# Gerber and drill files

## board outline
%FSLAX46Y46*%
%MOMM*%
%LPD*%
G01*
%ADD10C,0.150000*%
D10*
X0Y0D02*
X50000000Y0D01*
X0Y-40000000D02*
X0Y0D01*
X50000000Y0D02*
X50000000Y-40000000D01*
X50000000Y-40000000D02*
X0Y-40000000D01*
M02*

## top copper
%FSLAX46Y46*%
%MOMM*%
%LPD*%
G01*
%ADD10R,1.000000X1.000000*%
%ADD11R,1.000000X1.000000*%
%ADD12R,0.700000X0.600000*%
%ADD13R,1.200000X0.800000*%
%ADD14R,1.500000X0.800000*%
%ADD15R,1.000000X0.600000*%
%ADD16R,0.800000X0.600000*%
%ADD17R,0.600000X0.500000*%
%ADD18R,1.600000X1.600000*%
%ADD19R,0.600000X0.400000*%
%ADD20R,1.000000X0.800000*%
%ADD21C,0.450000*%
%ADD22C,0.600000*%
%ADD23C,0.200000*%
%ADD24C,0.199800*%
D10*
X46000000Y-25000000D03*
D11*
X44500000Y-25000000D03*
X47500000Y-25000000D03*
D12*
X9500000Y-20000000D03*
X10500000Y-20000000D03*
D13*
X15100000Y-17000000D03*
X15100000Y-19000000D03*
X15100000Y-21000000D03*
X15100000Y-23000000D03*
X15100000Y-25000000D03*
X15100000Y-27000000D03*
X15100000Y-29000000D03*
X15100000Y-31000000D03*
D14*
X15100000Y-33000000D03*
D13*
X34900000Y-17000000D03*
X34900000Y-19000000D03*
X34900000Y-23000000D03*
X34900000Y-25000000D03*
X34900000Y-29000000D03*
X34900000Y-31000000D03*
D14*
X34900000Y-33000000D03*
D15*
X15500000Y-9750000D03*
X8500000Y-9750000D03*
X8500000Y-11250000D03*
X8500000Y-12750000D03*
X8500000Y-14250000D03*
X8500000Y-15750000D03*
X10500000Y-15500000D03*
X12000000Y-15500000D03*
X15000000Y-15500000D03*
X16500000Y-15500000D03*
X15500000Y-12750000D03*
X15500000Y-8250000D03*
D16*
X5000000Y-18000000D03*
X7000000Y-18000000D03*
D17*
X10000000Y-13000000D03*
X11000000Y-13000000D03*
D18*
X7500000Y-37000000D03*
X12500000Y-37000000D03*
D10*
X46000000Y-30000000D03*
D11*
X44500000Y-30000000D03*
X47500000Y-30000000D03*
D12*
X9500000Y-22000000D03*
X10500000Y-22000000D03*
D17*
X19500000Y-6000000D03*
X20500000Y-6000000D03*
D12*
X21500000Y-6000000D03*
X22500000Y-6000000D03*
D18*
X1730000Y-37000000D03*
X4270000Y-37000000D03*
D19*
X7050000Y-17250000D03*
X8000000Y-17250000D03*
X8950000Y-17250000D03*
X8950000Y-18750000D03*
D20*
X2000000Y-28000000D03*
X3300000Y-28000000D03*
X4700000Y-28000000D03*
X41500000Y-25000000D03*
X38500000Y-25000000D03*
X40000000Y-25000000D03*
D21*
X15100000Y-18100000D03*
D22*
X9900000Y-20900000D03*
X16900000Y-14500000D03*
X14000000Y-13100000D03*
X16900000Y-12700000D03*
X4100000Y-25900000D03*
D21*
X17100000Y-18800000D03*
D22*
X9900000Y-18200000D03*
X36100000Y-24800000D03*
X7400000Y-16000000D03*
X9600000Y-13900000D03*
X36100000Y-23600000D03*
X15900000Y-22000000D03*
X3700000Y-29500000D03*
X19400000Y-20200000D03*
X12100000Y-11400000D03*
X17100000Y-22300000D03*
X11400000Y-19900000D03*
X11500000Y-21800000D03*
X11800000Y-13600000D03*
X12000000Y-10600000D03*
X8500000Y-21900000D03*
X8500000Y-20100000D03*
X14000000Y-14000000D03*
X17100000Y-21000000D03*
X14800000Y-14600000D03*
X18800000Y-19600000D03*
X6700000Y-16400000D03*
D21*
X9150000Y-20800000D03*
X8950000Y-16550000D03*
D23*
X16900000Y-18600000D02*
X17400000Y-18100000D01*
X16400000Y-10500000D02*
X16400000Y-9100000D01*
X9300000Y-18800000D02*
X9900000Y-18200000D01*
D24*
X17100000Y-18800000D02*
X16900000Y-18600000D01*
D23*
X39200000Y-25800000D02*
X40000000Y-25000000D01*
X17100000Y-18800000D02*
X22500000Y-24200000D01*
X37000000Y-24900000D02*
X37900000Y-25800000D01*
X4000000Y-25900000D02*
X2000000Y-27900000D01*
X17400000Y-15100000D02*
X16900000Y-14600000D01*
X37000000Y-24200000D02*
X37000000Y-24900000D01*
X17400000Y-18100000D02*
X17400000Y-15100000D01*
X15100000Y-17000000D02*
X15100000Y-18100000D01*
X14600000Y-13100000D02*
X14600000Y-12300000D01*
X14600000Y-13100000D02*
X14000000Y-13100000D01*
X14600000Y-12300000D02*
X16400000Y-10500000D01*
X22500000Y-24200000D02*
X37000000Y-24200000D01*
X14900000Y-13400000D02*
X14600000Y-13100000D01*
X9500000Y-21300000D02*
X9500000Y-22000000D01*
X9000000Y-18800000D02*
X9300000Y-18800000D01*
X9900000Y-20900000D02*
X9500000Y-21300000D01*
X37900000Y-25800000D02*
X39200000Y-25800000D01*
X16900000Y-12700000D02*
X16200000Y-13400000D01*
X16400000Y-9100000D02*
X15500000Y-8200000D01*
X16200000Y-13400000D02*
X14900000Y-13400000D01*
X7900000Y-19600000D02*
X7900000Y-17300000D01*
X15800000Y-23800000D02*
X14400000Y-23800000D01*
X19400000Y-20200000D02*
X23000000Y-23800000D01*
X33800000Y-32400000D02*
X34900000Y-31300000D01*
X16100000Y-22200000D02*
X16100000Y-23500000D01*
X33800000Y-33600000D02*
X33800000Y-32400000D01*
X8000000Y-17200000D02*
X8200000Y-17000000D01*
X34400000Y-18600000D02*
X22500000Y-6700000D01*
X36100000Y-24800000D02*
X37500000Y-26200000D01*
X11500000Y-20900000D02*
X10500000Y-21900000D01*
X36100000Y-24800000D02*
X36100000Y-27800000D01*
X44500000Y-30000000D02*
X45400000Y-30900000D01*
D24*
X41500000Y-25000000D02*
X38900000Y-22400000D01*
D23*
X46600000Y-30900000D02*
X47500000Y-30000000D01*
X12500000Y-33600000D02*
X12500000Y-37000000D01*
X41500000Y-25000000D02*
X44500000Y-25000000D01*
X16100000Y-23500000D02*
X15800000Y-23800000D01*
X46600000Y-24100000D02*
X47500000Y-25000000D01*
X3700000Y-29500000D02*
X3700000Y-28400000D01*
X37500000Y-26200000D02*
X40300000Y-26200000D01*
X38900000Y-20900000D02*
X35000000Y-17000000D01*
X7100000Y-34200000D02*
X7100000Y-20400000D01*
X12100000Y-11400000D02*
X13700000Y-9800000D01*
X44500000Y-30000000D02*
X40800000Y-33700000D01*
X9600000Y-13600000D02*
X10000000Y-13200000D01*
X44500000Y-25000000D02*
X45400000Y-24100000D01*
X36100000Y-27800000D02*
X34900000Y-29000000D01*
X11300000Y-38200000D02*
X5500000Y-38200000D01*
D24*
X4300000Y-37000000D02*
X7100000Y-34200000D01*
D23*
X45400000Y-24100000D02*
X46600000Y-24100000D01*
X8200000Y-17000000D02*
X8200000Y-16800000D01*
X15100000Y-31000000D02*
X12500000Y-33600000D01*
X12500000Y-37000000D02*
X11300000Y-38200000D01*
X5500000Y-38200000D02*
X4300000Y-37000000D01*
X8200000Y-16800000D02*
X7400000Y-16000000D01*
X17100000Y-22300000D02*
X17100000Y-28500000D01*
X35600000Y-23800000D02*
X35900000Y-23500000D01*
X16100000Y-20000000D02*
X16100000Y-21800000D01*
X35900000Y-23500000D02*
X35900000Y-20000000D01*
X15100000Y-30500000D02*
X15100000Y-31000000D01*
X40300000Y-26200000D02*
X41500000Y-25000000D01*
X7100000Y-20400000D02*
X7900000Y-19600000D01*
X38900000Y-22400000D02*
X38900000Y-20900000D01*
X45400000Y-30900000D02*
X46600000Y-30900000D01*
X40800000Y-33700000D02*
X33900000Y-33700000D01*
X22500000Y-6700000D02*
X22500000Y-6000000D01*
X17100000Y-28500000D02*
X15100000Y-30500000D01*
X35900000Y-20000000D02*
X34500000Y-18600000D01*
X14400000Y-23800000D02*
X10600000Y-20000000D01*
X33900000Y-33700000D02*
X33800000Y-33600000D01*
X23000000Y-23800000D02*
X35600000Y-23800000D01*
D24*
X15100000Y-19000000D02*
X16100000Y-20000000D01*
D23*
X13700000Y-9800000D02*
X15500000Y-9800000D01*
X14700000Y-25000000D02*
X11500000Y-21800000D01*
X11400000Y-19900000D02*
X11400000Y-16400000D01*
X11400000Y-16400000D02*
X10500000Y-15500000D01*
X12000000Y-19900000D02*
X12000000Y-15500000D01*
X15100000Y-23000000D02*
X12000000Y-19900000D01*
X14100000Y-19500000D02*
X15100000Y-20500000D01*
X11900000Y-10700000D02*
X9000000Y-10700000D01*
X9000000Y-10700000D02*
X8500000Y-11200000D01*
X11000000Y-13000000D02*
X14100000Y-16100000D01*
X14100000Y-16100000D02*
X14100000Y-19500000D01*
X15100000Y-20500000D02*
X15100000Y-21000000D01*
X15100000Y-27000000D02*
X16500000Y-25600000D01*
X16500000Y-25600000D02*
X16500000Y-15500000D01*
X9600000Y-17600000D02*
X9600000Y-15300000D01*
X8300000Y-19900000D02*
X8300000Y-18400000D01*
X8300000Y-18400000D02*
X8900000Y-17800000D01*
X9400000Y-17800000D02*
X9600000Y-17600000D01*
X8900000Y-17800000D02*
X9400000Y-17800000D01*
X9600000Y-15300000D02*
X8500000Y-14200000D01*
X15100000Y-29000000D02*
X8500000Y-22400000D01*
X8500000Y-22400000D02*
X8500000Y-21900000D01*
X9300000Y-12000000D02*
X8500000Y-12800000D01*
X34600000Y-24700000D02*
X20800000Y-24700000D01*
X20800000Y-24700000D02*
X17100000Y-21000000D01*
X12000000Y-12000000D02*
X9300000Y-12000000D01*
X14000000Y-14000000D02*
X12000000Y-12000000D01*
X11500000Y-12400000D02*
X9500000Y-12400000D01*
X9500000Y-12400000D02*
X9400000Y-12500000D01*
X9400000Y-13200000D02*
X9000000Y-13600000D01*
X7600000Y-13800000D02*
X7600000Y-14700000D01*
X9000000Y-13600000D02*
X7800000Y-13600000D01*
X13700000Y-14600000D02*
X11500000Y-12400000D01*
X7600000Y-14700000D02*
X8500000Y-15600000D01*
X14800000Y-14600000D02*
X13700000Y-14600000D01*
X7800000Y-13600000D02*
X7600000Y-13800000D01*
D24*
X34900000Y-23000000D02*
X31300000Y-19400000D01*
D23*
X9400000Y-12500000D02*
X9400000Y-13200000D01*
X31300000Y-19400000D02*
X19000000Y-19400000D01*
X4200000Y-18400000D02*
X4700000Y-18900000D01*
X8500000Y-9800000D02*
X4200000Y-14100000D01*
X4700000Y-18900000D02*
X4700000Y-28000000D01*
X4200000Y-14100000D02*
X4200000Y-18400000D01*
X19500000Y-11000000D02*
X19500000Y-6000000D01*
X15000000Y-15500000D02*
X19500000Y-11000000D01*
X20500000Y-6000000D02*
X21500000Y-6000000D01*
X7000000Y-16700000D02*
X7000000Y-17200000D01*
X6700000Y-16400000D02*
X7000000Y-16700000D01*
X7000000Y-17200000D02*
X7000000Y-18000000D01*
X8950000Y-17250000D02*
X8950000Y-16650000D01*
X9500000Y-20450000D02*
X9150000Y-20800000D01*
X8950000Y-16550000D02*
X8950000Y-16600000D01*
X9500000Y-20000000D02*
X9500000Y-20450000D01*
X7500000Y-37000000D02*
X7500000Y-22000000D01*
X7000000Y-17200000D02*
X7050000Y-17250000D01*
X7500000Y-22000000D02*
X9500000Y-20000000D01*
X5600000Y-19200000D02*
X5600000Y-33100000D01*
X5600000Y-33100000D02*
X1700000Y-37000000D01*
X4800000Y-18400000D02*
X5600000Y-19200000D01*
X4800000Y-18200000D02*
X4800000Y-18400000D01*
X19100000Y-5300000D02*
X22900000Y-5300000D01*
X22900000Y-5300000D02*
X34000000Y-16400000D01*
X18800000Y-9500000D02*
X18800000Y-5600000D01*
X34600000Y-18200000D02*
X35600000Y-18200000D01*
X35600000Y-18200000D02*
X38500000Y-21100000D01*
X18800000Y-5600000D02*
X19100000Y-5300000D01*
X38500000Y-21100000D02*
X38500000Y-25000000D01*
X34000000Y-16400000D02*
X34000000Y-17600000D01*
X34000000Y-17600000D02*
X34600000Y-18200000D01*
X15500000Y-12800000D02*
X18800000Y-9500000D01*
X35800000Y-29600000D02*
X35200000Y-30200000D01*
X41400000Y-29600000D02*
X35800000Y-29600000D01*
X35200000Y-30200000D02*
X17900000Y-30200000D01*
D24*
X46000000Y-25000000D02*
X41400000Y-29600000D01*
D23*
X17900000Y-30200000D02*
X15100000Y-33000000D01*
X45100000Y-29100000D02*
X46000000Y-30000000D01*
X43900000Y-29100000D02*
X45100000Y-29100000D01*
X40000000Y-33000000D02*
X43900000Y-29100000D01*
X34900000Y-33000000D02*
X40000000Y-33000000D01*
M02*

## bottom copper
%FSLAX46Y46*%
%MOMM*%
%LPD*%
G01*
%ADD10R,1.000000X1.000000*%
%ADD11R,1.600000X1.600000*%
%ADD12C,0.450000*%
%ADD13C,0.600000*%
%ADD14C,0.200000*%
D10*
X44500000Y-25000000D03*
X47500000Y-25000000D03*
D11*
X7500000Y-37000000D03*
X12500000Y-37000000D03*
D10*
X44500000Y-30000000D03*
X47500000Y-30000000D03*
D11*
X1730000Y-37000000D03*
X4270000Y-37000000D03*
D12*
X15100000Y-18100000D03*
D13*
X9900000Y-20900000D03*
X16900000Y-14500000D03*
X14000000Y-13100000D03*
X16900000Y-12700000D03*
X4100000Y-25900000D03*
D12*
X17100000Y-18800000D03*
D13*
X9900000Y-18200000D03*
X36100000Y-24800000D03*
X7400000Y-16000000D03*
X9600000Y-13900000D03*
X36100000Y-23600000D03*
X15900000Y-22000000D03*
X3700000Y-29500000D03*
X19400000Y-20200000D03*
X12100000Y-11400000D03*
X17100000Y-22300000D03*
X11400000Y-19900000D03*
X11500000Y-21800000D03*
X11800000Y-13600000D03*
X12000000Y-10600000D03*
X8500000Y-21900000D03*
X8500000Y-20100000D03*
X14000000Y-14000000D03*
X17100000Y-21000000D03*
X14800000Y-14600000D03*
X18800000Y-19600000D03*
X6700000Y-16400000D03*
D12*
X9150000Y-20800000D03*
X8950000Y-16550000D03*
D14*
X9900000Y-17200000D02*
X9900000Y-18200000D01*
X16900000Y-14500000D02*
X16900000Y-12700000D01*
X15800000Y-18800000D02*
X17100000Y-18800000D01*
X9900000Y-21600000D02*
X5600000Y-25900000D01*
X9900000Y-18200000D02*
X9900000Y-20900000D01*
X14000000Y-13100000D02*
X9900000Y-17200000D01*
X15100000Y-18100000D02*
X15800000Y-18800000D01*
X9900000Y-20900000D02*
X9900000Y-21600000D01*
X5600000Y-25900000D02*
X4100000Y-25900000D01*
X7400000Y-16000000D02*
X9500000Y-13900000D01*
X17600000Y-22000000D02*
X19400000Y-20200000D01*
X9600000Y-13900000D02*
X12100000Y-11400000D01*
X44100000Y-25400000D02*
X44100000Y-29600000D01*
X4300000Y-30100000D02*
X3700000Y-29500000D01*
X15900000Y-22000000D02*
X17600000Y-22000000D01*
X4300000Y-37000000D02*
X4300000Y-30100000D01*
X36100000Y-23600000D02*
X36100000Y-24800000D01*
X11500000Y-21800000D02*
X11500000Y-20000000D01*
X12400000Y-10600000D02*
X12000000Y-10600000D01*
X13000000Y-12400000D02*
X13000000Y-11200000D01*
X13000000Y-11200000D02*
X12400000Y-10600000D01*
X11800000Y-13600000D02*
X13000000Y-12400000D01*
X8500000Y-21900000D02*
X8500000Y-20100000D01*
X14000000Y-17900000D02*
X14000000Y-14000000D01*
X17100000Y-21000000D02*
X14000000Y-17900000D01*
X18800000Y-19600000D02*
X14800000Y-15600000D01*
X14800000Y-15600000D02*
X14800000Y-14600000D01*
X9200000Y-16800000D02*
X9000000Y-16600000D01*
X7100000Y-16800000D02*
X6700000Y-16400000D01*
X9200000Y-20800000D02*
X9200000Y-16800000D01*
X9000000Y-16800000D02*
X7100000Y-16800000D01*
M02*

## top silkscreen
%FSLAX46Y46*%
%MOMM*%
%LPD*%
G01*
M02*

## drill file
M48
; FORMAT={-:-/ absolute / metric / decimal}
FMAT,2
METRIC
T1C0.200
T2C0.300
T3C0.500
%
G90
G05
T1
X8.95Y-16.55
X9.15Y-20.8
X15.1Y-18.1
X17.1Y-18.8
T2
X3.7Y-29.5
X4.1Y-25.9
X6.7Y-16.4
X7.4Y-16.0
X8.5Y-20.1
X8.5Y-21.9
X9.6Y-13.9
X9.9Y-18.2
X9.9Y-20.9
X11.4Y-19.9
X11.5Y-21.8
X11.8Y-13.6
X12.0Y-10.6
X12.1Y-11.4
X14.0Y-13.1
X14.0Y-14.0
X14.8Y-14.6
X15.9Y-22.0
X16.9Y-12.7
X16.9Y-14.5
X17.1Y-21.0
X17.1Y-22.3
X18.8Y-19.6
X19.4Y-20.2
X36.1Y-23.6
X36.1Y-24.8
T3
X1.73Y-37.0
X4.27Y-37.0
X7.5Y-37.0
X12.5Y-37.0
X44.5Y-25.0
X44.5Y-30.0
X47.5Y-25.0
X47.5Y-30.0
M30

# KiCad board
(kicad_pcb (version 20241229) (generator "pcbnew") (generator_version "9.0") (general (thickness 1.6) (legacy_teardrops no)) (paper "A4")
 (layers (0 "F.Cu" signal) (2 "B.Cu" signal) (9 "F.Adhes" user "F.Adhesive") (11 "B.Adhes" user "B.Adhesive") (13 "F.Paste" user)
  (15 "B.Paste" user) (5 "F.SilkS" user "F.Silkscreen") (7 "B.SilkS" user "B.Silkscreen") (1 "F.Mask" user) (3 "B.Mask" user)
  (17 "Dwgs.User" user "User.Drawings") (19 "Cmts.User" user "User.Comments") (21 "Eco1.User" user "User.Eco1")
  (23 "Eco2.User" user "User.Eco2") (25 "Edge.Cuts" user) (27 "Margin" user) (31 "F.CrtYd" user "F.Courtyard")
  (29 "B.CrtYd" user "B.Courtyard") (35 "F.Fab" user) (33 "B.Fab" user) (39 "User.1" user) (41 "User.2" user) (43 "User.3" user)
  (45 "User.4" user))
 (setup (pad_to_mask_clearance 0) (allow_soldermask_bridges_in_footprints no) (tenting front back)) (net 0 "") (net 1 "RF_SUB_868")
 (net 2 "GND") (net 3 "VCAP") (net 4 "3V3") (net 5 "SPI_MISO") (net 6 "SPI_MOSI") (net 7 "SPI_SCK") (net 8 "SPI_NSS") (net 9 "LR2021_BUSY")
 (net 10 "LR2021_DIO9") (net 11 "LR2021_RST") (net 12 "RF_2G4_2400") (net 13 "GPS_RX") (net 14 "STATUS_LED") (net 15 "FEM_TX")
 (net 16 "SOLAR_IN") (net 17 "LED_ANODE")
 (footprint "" (layer "F.Cu") (at 46 25)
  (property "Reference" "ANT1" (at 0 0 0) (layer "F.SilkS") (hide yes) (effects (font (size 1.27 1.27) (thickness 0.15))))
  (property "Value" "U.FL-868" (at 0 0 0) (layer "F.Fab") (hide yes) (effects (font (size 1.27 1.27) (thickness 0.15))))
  (pad "1" smd rect (at 0 0) (size 1 1) (layers "F.Cu" "F.Mask") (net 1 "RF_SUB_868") (thermal_bridge_angle 45))
  (pad "2" thru_hole rect (at -1.5 0) (size 1 1) (drill 0.5) (layers "*.Cu" "*.Mask") (remove_unused_layers no) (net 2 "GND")
   (thermal_bridge_angle 45))
  (pad "3" thru_hole rect (at 1.5 0) (size 1 1) (drill 0.5) (layers "*.Cu" "*.Mask") (remove_unused_layers no) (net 2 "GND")
   (thermal_bridge_angle 45)))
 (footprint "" (layer "F.Cu") (at 10 20)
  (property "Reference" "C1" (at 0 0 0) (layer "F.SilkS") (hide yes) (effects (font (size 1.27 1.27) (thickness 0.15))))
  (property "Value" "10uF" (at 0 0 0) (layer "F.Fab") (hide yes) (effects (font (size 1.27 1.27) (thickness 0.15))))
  (pad "1" smd rect (at -0.5 0) (size 0.7 0.6) (layers "F.Cu" "F.Mask") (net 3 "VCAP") (thermal_bridge_angle 45))
  (pad "2" smd rect (at 0.5 0) (size 0.7 0.6) (layers "F.Cu" "F.Mask") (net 2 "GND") (thermal_bridge_angle 45)))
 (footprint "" (layer "F.Cu") (at 25 25)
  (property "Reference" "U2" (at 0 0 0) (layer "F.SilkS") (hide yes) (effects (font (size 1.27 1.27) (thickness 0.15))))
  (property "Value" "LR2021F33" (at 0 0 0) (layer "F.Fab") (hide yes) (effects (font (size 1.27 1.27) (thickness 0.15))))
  (pad "1" smd rect (at -9.9 -8) (size 1.2 0.8) (layers "F.Cu" "F.Mask") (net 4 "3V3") (thermal_bridge_angle 45))
  (pad "2" smd rect (at -9.9 -6) (size 1.2 0.8) (layers "F.Cu" "F.Mask") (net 2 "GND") (thermal_bridge_angle 45))
  (pad "3" smd rect (at -9.9 -4) (size 1.2 0.8) (layers "F.Cu" "F.Mask") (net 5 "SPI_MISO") (thermal_bridge_angle 45))
  (pad "4" smd rect (at -9.9 -2) (size 1.2 0.8) (layers "F.Cu" "F.Mask") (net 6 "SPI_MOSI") (thermal_bridge_angle 45))
  (pad "5" smd rect (at -9.9 0) (size 1.2 0.8) (layers "F.Cu" "F.Mask") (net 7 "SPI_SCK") (thermal_bridge_angle 45))
  (pad "6" smd rect (at -9.9 2) (size 1.2 0.8) (layers "F.Cu" "F.Mask") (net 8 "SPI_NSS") (thermal_bridge_angle 45))
  (pad "7" smd rect (at -9.9 4) (size 1.2 0.8) (layers "F.Cu" "F.Mask") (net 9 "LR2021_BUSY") (thermal_bridge_angle 45))
  (pad "8" smd rect (at -9.9 6) (size 1.2 0.8) (layers "F.Cu" "F.Mask") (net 2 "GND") (thermal_bridge_angle 45))
  (pad "9" smd rect (at -9.9 8) (size 1.5 0.8) (layers "F.Cu" "F.Mask") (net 1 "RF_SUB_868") (thermal_bridge_angle 45))
  (pad "10" smd rect (at 9.9 -8) (size 1.2 0.8) (layers "F.Cu" "F.Mask") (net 2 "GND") (thermal_bridge_angle 45))
  (pad "11" smd rect (at 9.9 -6) (size 1.2 0.8) (layers "F.Cu" "F.Mask") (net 2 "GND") (thermal_bridge_angle 45))
  (pad "13" smd rect (at 9.9 -2) (size 1.2 0.8) (layers "F.Cu" "F.Mask") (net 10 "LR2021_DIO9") (thermal_bridge_angle 45))
  (pad "14" smd rect (at 9.9 0) (size 1.2 0.8) (layers "F.Cu" "F.Mask") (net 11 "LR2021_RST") (thermal_bridge_angle 45))
  (pad "16" smd rect (at 9.9 4) (size 1.2 0.8) (layers "F.Cu" "F.Mask") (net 2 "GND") (thermal_bridge_angle 45))
  (pad "17" smd rect (at 9.9 6) (size 1.2 0.8) (layers "F.Cu" "F.Mask") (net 2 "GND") (thermal_bridge_angle 45))
  (pad "18" smd rect (at 9.9 8) (size 1.5 0.8) (layers "F.Cu" "F.Mask") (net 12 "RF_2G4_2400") (thermal_bridge_angle 45)))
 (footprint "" (layer "F.Cu") (at 12 12)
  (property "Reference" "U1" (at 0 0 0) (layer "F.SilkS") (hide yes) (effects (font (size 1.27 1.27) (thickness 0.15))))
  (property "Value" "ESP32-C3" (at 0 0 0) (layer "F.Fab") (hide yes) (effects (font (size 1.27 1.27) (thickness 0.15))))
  (pad "GND" smd rect (at 3.5 -2.25) (size 1 0.6) (layers "F.Cu" "F.Mask") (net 2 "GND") (thermal_bridge_angle 45))
  (pad "GPIO1" smd rect (at -3.5 -2.25) (size 1 0.6) (layers "F.Cu" "F.Mask") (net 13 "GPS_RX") (thermal_bridge_angle 45))
  (pad "GPIO2" smd rect (at -3.5 -0.75) (size 1 0.6) (layers "F.Cu" "F.Mask") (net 5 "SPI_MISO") (thermal_bridge_angle 45))
  (pad "GPIO3" smd rect (at -3.5 0.75) (size 1 0.6) (layers "F.Cu" "F.Mask") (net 11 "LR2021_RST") (thermal_bridge_angle 45))
  (pad "GPIO4" smd rect (at -3.5 2.25) (size 1 0.6) (layers "F.Cu" "F.Mask") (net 9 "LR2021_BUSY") (thermal_bridge_angle 45))
  (pad "GPIO5" smd rect (at -3.5 3.75) (size 1 0.6) (layers "F.Cu" "F.Mask") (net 10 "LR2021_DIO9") (thermal_bridge_angle 45))
  (pad "GPIO6" smd rect (at -1.5 3.5) (size 1 0.6) (layers "F.Cu" "F.Mask") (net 7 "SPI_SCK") (thermal_bridge_angle 45))
  (pad "GPIO7" smd rect (at 0 3.5) (size 1 0.6) (layers "F.Cu" "F.Mask") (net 6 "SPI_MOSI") (thermal_bridge_angle 45))
  (pad "GPIO9" smd rect (at 3 3.5) (size 1 0.6) (layers "F.Cu" "F.Mask") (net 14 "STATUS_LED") (thermal_bridge_angle 45))
  (pad "GPIO10" smd rect (at 4.5 3.5) (size 1 0.6) (layers "F.Cu" "F.Mask") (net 8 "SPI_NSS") (thermal_bridge_angle 45))
  (pad "GPIO19" smd rect (at 3.5 0.75) (size 1 0.6) (layers "F.Cu" "F.Mask") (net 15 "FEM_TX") (thermal_bridge_angle 45))
  (pad "VCC" smd rect (at 3.5 -3.75) (size 1 0.6) (layers "F.Cu" "F.Mask") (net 4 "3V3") (thermal_bridge_angle 45)))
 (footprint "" (layer "F.Cu") (at 6 18)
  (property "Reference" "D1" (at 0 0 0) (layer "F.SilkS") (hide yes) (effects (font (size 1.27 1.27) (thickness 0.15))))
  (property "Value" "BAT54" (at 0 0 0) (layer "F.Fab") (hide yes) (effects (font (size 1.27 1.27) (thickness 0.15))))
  (pad "A" smd rect (at -1 0) (size 0.8 0.6) (layers "F.Cu" "F.Mask") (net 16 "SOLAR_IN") (thermal_bridge_angle 45))
  (pad "K" smd rect (at 1 0) (size 0.8 0.6) (layers "F.Cu" "F.Mask") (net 3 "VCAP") (thermal_bridge_angle 45)))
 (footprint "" (layer "F.Cu") (at 10.5 13)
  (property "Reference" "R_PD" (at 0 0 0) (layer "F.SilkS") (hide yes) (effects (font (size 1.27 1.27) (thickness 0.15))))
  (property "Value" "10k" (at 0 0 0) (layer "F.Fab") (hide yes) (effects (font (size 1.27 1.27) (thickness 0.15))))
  (pad "1" smd rect (at -0.5 0) (size 0.6 0.5) (layers "F.Cu" "F.Mask") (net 2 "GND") (thermal_bridge_angle 45))
  (pad "2" smd rect (at 0.5 0) (size 0.6 0.5) (layers "F.Cu" "F.Mask") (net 5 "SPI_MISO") (thermal_bridge_angle 45)))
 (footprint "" (layer "F.Cu") (at 10 37)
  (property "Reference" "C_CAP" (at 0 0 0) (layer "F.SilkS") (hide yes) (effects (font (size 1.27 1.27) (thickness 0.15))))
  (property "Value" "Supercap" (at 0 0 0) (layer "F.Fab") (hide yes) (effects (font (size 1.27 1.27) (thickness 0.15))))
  (pad "1" thru_hole rect (at -2.5 0) (size 1.6 1.6) (drill 0.5) (layers "*.Cu" "*.Mask") (remove_unused_layers no) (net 3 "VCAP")
   (thermal_bridge_angle 45))
  (pad "2" thru_hole rect (at 2.5 0) (size 1.6 1.6) (drill 0.5) (layers "*.Cu" "*.Mask") (remove_unused_layers no) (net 2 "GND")
   (thermal_bridge_angle 45)))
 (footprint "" (layer "F.Cu") (at 46 30)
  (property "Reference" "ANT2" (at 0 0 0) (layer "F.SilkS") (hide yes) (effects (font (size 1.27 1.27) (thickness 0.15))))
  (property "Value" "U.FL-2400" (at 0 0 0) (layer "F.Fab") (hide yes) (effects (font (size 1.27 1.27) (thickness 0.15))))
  (pad "1" smd rect (at 0 0) (size 1 1) (layers "F.Cu" "F.Mask") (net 12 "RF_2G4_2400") (thermal_bridge_angle 45))
  (pad "2" thru_hole rect (at -1.5 0) (size 1 1) (drill 0.5) (layers "*.Cu" "*.Mask") (remove_unused_layers no) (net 2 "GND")
   (thermal_bridge_angle 45))
  (pad "3" thru_hole rect (at 1.5 0) (size 1 1) (drill 0.5) (layers "*.Cu" "*.Mask") (remove_unused_layers no) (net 2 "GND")
   (thermal_bridge_angle 45)))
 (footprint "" (layer "F.Cu") (at 10 22)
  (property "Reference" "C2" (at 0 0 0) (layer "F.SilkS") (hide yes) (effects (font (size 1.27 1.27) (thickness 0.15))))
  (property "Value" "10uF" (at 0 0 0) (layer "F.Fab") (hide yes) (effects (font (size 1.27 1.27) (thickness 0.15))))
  (pad "1" smd rect (at -0.5 0) (size 0.7 0.6) (layers "F.Cu" "F.Mask") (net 4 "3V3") (thermal_bridge_angle 45))
  (pad "2" smd rect (at 0.5 0) (size 0.7 0.6) (layers "F.Cu" "F.Mask") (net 2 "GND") (thermal_bridge_angle 45)))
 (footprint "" (layer "F.Cu") (at 20 6)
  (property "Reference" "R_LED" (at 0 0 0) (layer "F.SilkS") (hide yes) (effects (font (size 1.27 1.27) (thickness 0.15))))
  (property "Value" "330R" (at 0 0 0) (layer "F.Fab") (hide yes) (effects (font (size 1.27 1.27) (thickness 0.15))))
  (pad "1" smd rect (at -0.5 0) (size 0.6 0.5) (layers "F.Cu" "F.Mask") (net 14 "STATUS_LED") (thermal_bridge_angle 45))
  (pad "2" smd rect (at 0.5 0) (size 0.6 0.5) (layers "F.Cu" "F.Mask") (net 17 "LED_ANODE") (thermal_bridge_angle 45)))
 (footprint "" (layer "F.Cu") (at 22 6)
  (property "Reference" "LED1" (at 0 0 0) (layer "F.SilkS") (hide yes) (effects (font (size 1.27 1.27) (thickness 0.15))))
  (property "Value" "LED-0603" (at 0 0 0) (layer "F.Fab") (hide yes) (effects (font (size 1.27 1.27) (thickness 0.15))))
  (pad "A" smd rect (at -0.5 0) (size 0.7 0.6) (layers "F.Cu" "F.Mask") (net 17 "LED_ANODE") (thermal_bridge_angle 45))
  (pad "K" smd rect (at 0.5 0) (size 0.7 0.6) (layers "F.Cu" "F.Mask") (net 2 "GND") (thermal_bridge_angle 45)))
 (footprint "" (layer "F.Cu") (at 3 37)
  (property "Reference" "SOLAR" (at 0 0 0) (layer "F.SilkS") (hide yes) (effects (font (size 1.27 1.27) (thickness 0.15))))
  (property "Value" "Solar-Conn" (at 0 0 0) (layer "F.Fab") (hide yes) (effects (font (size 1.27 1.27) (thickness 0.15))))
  (pad "1" thru_hole rect (at -1.27 0) (size 1.6 1.6) (drill 0.5) (layers "*.Cu" "*.Mask") (remove_unused_layers no) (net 16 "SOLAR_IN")
   (thermal_bridge_angle 45))
  (pad "2" thru_hole rect (at 1.27 0) (size 1.6 1.6) (drill 0.5) (layers "*.Cu" "*.Mask") (remove_unused_layers no) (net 2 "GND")
   (thermal_bridge_angle 45)))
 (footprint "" (layer "F.Cu") (at 8 18)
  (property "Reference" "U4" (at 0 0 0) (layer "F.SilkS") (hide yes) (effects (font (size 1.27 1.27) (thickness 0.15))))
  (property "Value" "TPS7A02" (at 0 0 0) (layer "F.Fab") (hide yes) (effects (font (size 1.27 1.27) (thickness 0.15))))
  (pad "1" smd rect (at -0.95 -0.75) (size 0.6 0.4) (layers "F.Cu" "F.Mask") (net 3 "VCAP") (thermal_bridge_angle 45))
  (pad "2" smd rect (at 0 -0.75) (size 0.6 0.4) (layers "F.Cu" "F.Mask") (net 2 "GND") (thermal_bridge_angle 45))
  (pad "3" smd rect (at 0.95 -0.75) (size 0.6 0.4) (layers "F.Cu" "F.Mask") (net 3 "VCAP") (thermal_bridge_angle 45))
  (pad "4" smd rect (at 0.95 0.75) (size 0.6 0.4) (layers "F.Cu" "F.Mask") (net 4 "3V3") (thermal_bridge_angle 45)))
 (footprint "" (layer "F.Cu") (at 4 28)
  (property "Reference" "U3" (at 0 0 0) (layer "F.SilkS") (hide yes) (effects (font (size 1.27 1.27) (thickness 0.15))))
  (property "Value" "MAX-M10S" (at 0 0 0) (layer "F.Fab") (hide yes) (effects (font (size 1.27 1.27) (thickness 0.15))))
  (pad "1" smd rect (at -2 0) (size 1 0.8) (layers "F.Cu" "F.Mask") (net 4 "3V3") (thermal_bridge_angle 45))
  (pad "2" smd rect (at -0.7 0) (size 1 0.8) (layers "F.Cu" "F.Mask") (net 2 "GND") (thermal_bridge_angle 45))
  (pad "3" smd rect (at 0.7 0) (size 1 0.8) (layers "F.Cu" "F.Mask") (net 13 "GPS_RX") (thermal_bridge_angle 45)))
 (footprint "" (layer "F.Cu") (at 40 25)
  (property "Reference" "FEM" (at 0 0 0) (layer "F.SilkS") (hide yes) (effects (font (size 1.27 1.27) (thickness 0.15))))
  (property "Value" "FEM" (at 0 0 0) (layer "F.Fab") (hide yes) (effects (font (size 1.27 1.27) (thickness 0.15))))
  (pad "GND" smd rect (at 1.5 0) (size 1 0.8) (layers "F.Cu" "F.Mask") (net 2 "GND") (thermal_bridge_angle 45))
  (pad "TX" smd rect (at -1.5 0) (size 1 0.8) (layers "F.Cu" "F.Mask") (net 15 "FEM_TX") (thermal_bridge_angle 45))
  (pad "VCC" smd rect (at 0 0) (size 1 0.8) (layers "F.Cu" "F.Mask") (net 4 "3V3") (thermal_bridge_angle 45)))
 (gr_line (start 0 0) (end 50 0) (stroke (width 0.15) (type default)) (layer "Edge.Cuts"))
 (gr_line (start 0 40) (end 0 0) (stroke (width 0.15) (type default)) (layer "Edge.Cuts"))
 (gr_line (start 50 0) (end 50 40) (stroke (width 0.15) (type default)) (layer "Edge.Cuts"))
 (gr_line (start 50 40) (end 0 40) (stroke (width 0.15) (type default)) (layer "Edge.Cuts"))
 (segment (start 16.9 18.6) (end 17.4 18.1) (width 0.2) (layer "F.Cu") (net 4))
 (segment (start 16.4 10.5) (end 16.4 9.1) (width 0.2) (layer "F.Cu") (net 4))
 (segment (start 9.3 18.8) (end 9.9 18.2) (width 0.2) (layer "F.Cu") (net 4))
 (segment (start 17.1 18.8) (end 16.9 18.6) (width 0.1998) (layer "F.Cu") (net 4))
 (segment (start 39.2 25.8) (end 40 25) (width 0.2) (layer "F.Cu") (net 4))
 (segment (start 17.1 18.8) (end 22.5 24.2) (width 0.2) (layer "F.Cu") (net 4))
 (segment (start 37 24.9) (end 37.9 25.8) (width 0.2) (layer "F.Cu") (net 4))
 (segment (start 4 25.9) (end 2 27.9) (width 0.2) (layer "F.Cu") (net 4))
 (segment (start 17.4 15.1) (end 16.9 14.6) (width 0.2) (layer "F.Cu") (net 4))
 (segment (start 37 24.2) (end 37 24.9) (width 0.2) (layer "F.Cu") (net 4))
 (segment (start 17.4 18.1) (end 17.4 15.1) (width 0.2) (layer "F.Cu") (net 4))
 (segment (start 15.1 17) (end 15.1 18.1) (width 0.2) (layer "F.Cu") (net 4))
 (segment (start 14.6 13.1) (end 14.6 12.3) (width 0.2) (layer "F.Cu") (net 4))
 (segment (start 14.6 13.1) (end 14 13.1) (width 0.2) (layer "F.Cu") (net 4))
 (segment (start 14.6 12.3) (end 16.4 10.5) (width 0.2) (layer "F.Cu") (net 4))
 (segment (start 22.5 24.2) (end 37 24.2) (width 0.2) (layer "F.Cu") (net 4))
 (segment (start 14.9 13.4) (end 14.6 13.1) (width 0.2) (layer "F.Cu") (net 4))
 (segment (start 9.5 21.3) (end 9.5 22) (width 0.2) (layer "F.Cu") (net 4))
 (segment (start 9 18.8) (end 9.3 18.8) (width 0.2) (layer "F.Cu") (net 4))
 (segment (start 9.9 20.9) (end 9.5 21.3) (width 0.2) (layer "F.Cu") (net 4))
 (segment (start 37.9 25.8) (end 39.2 25.8) (width 0.2) (layer "F.Cu") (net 4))
 (segment (start 16.9 12.7) (end 16.2 13.4) (width 0.2) (layer "F.Cu") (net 4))
 (segment (start 16.4 9.1) (end 15.5 8.2) (width 0.2) (layer "F.Cu") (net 4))
 (segment (start 16.2 13.4) (end 14.9 13.4) (width 0.2) (layer "F.Cu") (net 4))
 (via (at 15.1 18.1) (size 0.45) (drill 0.2) (layers "F.Cu" "B.Cu") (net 4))
 (via (at 9.9 20.9) (size 0.6) (drill 0.3) (layers "F.Cu" "B.Cu") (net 4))
 (via (at 16.9 14.5) (size 0.6) (drill 0.3) (layers "F.Cu" "B.Cu") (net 4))
 (via (at 14 13.1) (size 0.6) (drill 0.3) (layers "F.Cu" "B.Cu") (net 4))
 (via (at 16.9 12.7) (size 0.6) (drill 0.3) (layers "F.Cu" "B.Cu") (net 4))
 (via (at 4.1 25.9) (size 0.6) (drill 0.3) (layers "F.Cu" "B.Cu") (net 4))
 (via (at 17.1 18.8) (size 0.45) (drill 0.2) (layers "F.Cu" "B.Cu") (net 4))
 (via (at 9.9 18.2) (size 0.6) (drill 0.3) (layers "F.Cu" "B.Cu") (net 4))
 (segment (start 9.9 17.2) (end 9.9 18.2) (width 0.2) (layer "B.Cu") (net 4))
 (segment (start 16.9 14.5) (end 16.9 12.7) (width 0.2) (layer "B.Cu") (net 4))
 (segment (start 15.8 18.8) (end 17.1 18.8) (width 0.2) (layer "B.Cu") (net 4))
 (segment (start 9.9 21.6) (end 5.6 25.9) (width 0.2) (layer "B.Cu") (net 4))
 (segment (start 9.9 18.2) (end 9.9 20.9) (width 0.2) (layer "B.Cu") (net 4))
 (segment (start 14 13.1) (end 9.9 17.2) (width 0.2) (layer "B.Cu") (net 4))
 (segment (start 15.1 18.1) (end 15.8 18.8) (width 0.2) (layer "B.Cu") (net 4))
 (segment (start 9.9 20.9) (end 9.9 21.6) (width 0.2) (layer "B.Cu") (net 4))
 (segment (start 5.6 25.9) (end 4.1 25.9) (width 0.2) (layer "B.Cu") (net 4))
 (segment (start 7.9 19.6) (end 7.9 17.3) (width 0.2) (layer "F.Cu") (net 2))
 (segment (start 15.8 23.8) (end 14.4 23.8) (width 0.2) (layer "F.Cu") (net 2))
 (segment (start 19.4 20.2) (end 23 23.8) (width 0.2) (layer "F.Cu") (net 2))
 (segment (start 33.8 32.4) (end 34.9 31.3) (width 0.2) (layer "F.Cu") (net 2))
 (segment (start 16.1 22.2) (end 16.1 23.5) (width 0.2) (layer "F.Cu") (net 2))
 (segment (start 33.8 33.6) (end 33.8 32.4) (width 0.2) (layer "F.Cu") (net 2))
 (segment (start 8 17.2) (end 8.2 17) (width 0.2) (layer "F.Cu") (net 2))
 (segment (start 34.4 18.6) (end 22.5 6.7) (width 0.2) (layer "F.Cu") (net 2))
 (segment (start 36.1 24.8) (end 37.5 26.2) (width 0.2) (layer "F.Cu") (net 2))
 (segment (start 11.5 20.9) (end 10.5 21.9) (width 0.2) (layer "F.Cu") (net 2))
 (segment (start 36.1 24.8) (end 36.1 27.8) (width 0.2) (layer "F.Cu") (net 2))
 (segment (start 44.5 30) (end 45.4 30.9) (width 0.2) (layer "F.Cu") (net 2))
 (segment (start 41.5 25) (end 38.9 22.4) (width 0.1998) (layer "F.Cu") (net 2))
 (segment (start 46.6 30.9) (end 47.5 30) (width 0.2) (layer "F.Cu") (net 2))
 (segment (start 12.5 33.6) (end 12.5 37) (width 0.2) (layer "F.Cu") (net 2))
 (segment (start 41.5 25) (end 44.5 25) (width 0.2) (layer "F.Cu") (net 2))
 (segment (start 16.1 23.5) (end 15.8 23.8) (width 0.2) (layer "F.Cu") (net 2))
 (segment (start 46.6 24.1) (end 47.5 25) (width 0.2) (layer "F.Cu") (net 2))
 (segment (start 3.7 29.5) (end 3.7 28.4) (width 0.2) (layer "F.Cu") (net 2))
 (segment (start 37.5 26.2) (end 40.3 26.2) (width 0.2) (layer "F.Cu") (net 2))
 (segment (start 38.9 20.9) (end 35 17) (width 0.2) (layer "F.Cu") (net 2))
 (segment (start 7.1 34.2) (end 7.1 20.4) (width 0.2) (layer "F.Cu") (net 2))
 (segment (start 12.1 11.4) (end 13.7 9.8) (width 0.2) (layer "F.Cu") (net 2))
 (segment (start 44.5 30) (end 40.8 33.7) (width 0.2) (layer "F.Cu") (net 2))
 (segment (start 9.6 13.6) (end 10 13.2) (width 0.2) (layer "F.Cu") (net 2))
 (segment (start 44.5 25) (end 45.4 24.1) (width 0.2) (layer "F.Cu") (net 2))
 (segment (start 36.1 27.8) (end 34.9 29) (width 0.2) (layer "F.Cu") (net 2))
 (segment (start 11.3 38.2) (end 5.5 38.2) (width 0.2) (layer "F.Cu") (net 2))
 (segment (start 4.3 37) (end 7.1 34.2) (width 0.1998) (layer "F.Cu") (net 2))
 (segment (start 45.4 24.1) (end 46.6 24.1) (width 0.2) (layer "F.Cu") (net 2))
 (segment (start 8.2 17) (end 8.2 16.8) (width 0.2) (layer "F.Cu") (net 2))
 (segment (start 15.1 31) (end 12.5 33.6) (width 0.2) (layer "F.Cu") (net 2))
 (segment (start 12.5 37) (end 11.3 38.2) (width 0.2) (layer "F.Cu") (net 2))
 (segment (start 5.5 38.2) (end 4.3 37) (width 0.2) (layer "F.Cu") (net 2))
 (segment (start 8.2 16.8) (end 7.4 16) (width 0.2) (layer "F.Cu") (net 2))
 (segment (start 17.1 22.3) (end 17.1 28.5) (width 0.2) (layer "F.Cu") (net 2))
 (segment (start 35.6 23.8) (end 35.9 23.5) (width 0.2) (layer "F.Cu") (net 2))
 (segment (start 16.1 20) (end 16.1 21.8) (width 0.2) (layer "F.Cu") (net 2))
 (segment (start 35.9 23.5) (end 35.9 20) (width 0.2) (layer "F.Cu") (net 2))
 (segment (start 15.1 30.5) (end 15.1 31) (width 0.2) (layer "F.Cu") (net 2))
 (segment (start 40.3 26.2) (end 41.5 25) (width 0.2) (layer "F.Cu") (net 2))
 (segment (start 7.1 20.4) (end 7.9 19.6) (width 0.2) (layer "F.Cu") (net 2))
 (segment (start 38.9 22.4) (end 38.9 20.9) (width 0.2) (layer "F.Cu") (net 2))
 (segment (start 45.4 30.9) (end 46.6 30.9) (width 0.2) (layer "F.Cu") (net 2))
 (segment (start 40.8 33.7) (end 33.9 33.7) (width 0.2) (layer "F.Cu") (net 2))
 (segment (start 22.5 6.7) (end 22.5 6) (width 0.2) (layer "F.Cu") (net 2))
 (segment (start 17.1 28.5) (end 15.1 30.5) (width 0.2) (layer "F.Cu") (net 2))
 (segment (start 35.9 20) (end 34.5 18.6) (width 0.2) (layer "F.Cu") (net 2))
 (segment (start 14.4 23.8) (end 10.6 20) (width 0.2) (layer "F.Cu") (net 2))
 (segment (start 33.9 33.7) (end 33.8 33.6) (width 0.2) (layer "F.Cu") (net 2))
 (segment (start 23 23.8) (end 35.6 23.8) (width 0.2) (layer "F.Cu") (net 2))
 (segment (start 15.1 19) (end 16.1 20) (width 0.1998) (layer "F.Cu") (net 2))
 (segment (start 13.7 9.8) (end 15.5 9.8) (width 0.2) (layer "F.Cu") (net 2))
 (via (at 36.1 24.8) (size 0.6) (drill 0.3) (layers "F.Cu" "B.Cu") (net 2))
 (via (at 7.4 16) (size 0.6) (drill 0.3) (layers "F.Cu" "B.Cu") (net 2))
 (via (at 9.6 13.9) (size 0.6) (drill 0.3) (layers "F.Cu" "B.Cu") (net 2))
 (via (at 36.1 23.6) (size 0.6) (drill 0.3) (layers "F.Cu" "B.Cu") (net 2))
 (via (at 15.9 22) (size 0.6) (drill 0.3) (layers "F.Cu" "B.Cu") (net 2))
 (via (at 3.7 29.5) (size 0.6) (drill 0.3) (layers "F.Cu" "B.Cu") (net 2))
 (via (at 19.4 20.2) (size 0.6) (drill 0.3) (layers "F.Cu" "B.Cu") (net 2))
 (via (at 12.1 11.4) (size 0.6) (drill 0.3) (layers "F.Cu" "B.Cu") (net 2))
 (via (at 17.1 22.3) (size 0.6) (drill 0.3) (layers "F.Cu" "B.Cu") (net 2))
 (segment (start 7.4 16) (end 9.5 13.9) (width 0.2) (layer "B.Cu") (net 2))
 (segment (start 17.6 22) (end 19.4 20.2) (width 0.2) (layer "B.Cu") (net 2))
 (segment (start 9.6 13.9) (end 12.1 11.4) (width 0.2) (layer "B.Cu") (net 2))
 (segment (start 44.1 25.4) (end 44.1 29.6) (width 0.2) (layer "B.Cu") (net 2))
 (segment (start 4.3 30.1) (end 3.7 29.5) (width 0.2) (layer "B.Cu") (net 2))
 (segment (start 15.9 22) (end 17.6 22) (width 0.2) (layer "B.Cu") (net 2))
 (segment (start 4.3 37) (end 4.3 30.1) (width 0.2) (layer "B.Cu") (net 2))
 (segment (start 36.1 23.6) (end 36.1 24.8) (width 0.2) (layer "B.Cu") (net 2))
 (segment (start 14.7 25) (end 11.5 21.8) (width 0.2) (layer "F.Cu") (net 7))
 (segment (start 11.4 19.9) (end 11.4 16.4) (width 0.2) (layer "F.Cu") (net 7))
 (segment (start 11.4 16.4) (end 10.5 15.5) (width 0.2) (layer "F.Cu") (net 7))
 (via (at 11.4 19.9) (size 0.6) (drill 0.3) (layers "F.Cu" "B.Cu") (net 7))
 (via (at 11.5 21.8) (size 0.6) (drill 0.3) (layers "F.Cu" "B.Cu") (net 7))
 (segment (start 11.5 21.8) (end 11.5 20) (width 0.2) (layer "B.Cu") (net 7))
 (segment (start 12 19.9) (end 12 15.5) (width 0.2) (layer "F.Cu") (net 6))
 (segment (start 15.1 23) (end 12 19.9) (width 0.2) (layer "F.Cu") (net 6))
 (segment (start 14.1 19.5) (end 15.1 20.5) (width 0.2) (layer "F.Cu") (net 5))
 (segment (start 11.9 10.7) (end 9 10.7) (width 0.2) (layer "F.Cu") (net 5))
 (segment (start 9 10.7) (end 8.5 11.2) (width 0.2) (layer "F.Cu") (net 5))
 (segment (start 11 13) (end 14.1 16.1) (width 0.2) (layer "F.Cu") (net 5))
 (segment (start 14.1 16.1) (end 14.1 19.5) (width 0.2) (layer "F.Cu") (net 5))
 (segment (start 15.1 20.5) (end 15.1 21) (width 0.2) (layer "F.Cu") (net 5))
 (via (at 11.8 13.6) (size 0.6) (drill 0.3) (layers "F.Cu" "B.Cu") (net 5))
 (via (at 12 10.6) (size 0.6) (drill 0.3) (layers "F.Cu" "B.Cu") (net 5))
 (segment (start 12.4 10.6) (end 12 10.6) (width 0.2) (layer "B.Cu") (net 5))
 (segment (start 13 12.4) (end 13 11.2) (width 0.2) (layer "B.Cu") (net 5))
 (segment (start 13 11.2) (end 12.4 10.6) (width 0.2) (layer "B.Cu") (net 5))
 (segment (start 11.8 13.6) (end 13 12.4) (width 0.2) (layer "B.Cu") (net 5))
 (segment (start 15.1 27) (end 16.5 25.6) (width 0.2) (layer "F.Cu") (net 8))
 (segment (start 16.5 25.6) (end 16.5 15.5) (width 0.2) (layer "F.Cu") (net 8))
 (segment (start 9.6 17.6) (end 9.6 15.3) (width 0.2) (layer "F.Cu") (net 9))
 (segment (start 8.3 19.9) (end 8.3 18.4) (width 0.2) (layer "F.Cu") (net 9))
 (segment (start 8.3 18.4) (end 8.9 17.8) (width 0.2) (layer "F.Cu") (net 9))
 (segment (start 9.4 17.8) (end 9.6 17.6) (width 0.2) (layer "F.Cu") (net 9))
 (segment (start 8.9 17.8) (end 9.4 17.8) (width 0.2) (layer "F.Cu") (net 9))
 (segment (start 9.6 15.3) (end 8.5 14.2) (width 0.2) (layer "F.Cu") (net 9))
 (segment (start 15.1 29) (end 8.5 22.4) (width 0.2) (layer "F.Cu") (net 9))
 (segment (start 8.5 22.4) (end 8.5 21.9) (width 0.2) (layer "F.Cu") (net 9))
 (via (at 8.5 21.9) (size 0.6) (drill 0.3) (layers "F.Cu" "B.Cu") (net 9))
 (via (at 8.5 20.1) (size 0.6) (drill 0.3) (layers "F.Cu" "B.Cu") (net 9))
 (segment (start 8.5 21.9) (end 8.5 20.1) (width 0.2) (layer "B.Cu") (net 9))
 (segment (start 9.3 12) (end 8.5 12.8) (width 0.2) (layer "F.Cu") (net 11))
 (segment (start 34.6 24.7) (end 20.8 24.7) (width 0.2) (layer "F.Cu") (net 11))
 (segment (start 20.8 24.7) (end 17.1 21) (width 0.2) (layer "F.Cu") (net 11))
 (segment (start 12 12) (end 9.3 12) (width 0.2) (layer "F.Cu") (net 11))
 (segment (start 14 14) (end 12 12) (width 0.2) (layer "F.Cu") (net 11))
 (via (at 14 14) (size 0.6) (drill 0.3) (layers "F.Cu" "B.Cu") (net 11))
 (via (at 17.1 21) (size 0.6) (drill 0.3) (layers "F.Cu" "B.Cu") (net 11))
 (segment (start 14 17.9) (end 14 14) (width 0.2) (layer "B.Cu") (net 11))
 (segment (start 17.1 21) (end 14 17.9) (width 0.2) (layer "B.Cu") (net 11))
 (segment (start 11.5 12.4) (end 9.5 12.4) (width 0.2) (layer "F.Cu") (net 10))
 (segment (start 9.5 12.4) (end 9.4 12.5) (width 0.2) (layer "F.Cu") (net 10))
 (segment (start 9.4 13.2) (end 9 13.6) (width 0.2) (layer "F.Cu") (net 10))
 (segment (start 7.6 13.8) (end 7.6 14.7) (width 0.2) (layer "F.Cu") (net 10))
 (segment (start 9 13.6) (end 7.8 13.6) (width 0.2) (layer "F.Cu") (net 10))
 (segment (start 13.7 14.6) (end 11.5 12.4) (width 0.2) (layer "F.Cu") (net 10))
 (segment (start 7.6 14.7) (end 8.5 15.6) (width 0.2) (layer "F.Cu") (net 10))
 (segment (start 14.8 14.6) (end 13.7 14.6) (width 0.2) (layer "F.Cu") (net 10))
 (segment (start 7.8 13.6) (end 7.6 13.8) (width 0.2) (layer "F.Cu") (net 10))
 (segment (start 34.9 23) (end 31.3 19.4) (width 0.1998) (layer "F.Cu") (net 10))
 (segment (start 9.4 12.5) (end 9.4 13.2) (width 0.2) (layer "F.Cu") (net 10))
 (segment (start 31.3 19.4) (end 19 19.4) (width 0.2) (layer "F.Cu") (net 10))
 (via (at 14.8 14.6) (size 0.6) (drill 0.3) (layers "F.Cu" "B.Cu") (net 10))
 (via (at 18.8 19.6) (size 0.6) (drill 0.3) (layers "F.Cu" "B.Cu") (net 10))
 (segment (start 18.8 19.6) (end 14.8 15.6) (width 0.2) (layer "B.Cu") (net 10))
 (segment (start 14.8 15.6) (end 14.8 14.6) (width 0.2) (layer "B.Cu") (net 10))
 (segment (start 4.2 18.4) (end 4.7 18.9) (width 0.2) (layer "F.Cu") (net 13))
 (segment (start 8.5 9.8) (end 4.2 14.1) (width 0.2) (layer "F.Cu") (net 13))
 (segment (start 4.7 18.9) (end 4.7 28) (width 0.2) (layer "F.Cu") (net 13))
 (segment (start 4.2 14.1) (end 4.2 18.4) (width 0.2) (layer "F.Cu") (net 13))
 (segment (start 19.5 11) (end 19.5 6) (width 0.2) (layer "F.Cu") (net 14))
 (segment (start 15 15.5) (end 19.5 11) (width 0.2) (layer "F.Cu") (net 14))
 (segment (start 20.5 6) (end 21.5 6) (width 0.2) (layer "F.Cu") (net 17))
 (segment (start 7 16.7) (end 7 17.2) (width 0.2) (layer "F.Cu") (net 3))
 (segment (start 6.7 16.4) (end 7 16.7) (width 0.2) (layer "F.Cu") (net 3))
 (segment (start 7 17.2) (end 7 18) (width 0.2) (layer "F.Cu") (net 3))
 (segment (start 8.95 17.25) (end 8.95 16.65) (width 0.2) (layer "F.Cu") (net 3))
 (segment (start 9.5 20.45) (end 9.15 20.8) (width 0.2) (layer "F.Cu") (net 3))
 (segment (start 8.95 16.55) (end 8.95 16.6) (width 0.2) (layer "F.Cu") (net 3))
 (segment (start 9.5 20) (end 9.5 20.45) (width 0.2) (layer "F.Cu") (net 3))
 (segment (start 7.5 37) (end 7.5 22) (width 0.2) (layer "F.Cu") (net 3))
 (segment (start 7 17.2) (end 7.05 17.25) (width 0.2) (layer "F.Cu") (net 3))
 (segment (start 7.5 22) (end 9.5 20) (width 0.2) (layer "F.Cu") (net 3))
 (via (at 6.7 16.4) (size 0.6) (drill 0.3) (layers "F.Cu" "B.Cu") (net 3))
 (via (at 9.15 20.8) (size 0.45) (drill 0.2) (layers "F.Cu" "B.Cu") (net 3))
 (via (at 8.95 16.55) (size 0.45) (drill 0.2) (layers "F.Cu" "B.Cu") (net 3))
 (segment (start 9.2 16.8) (end 9 16.6) (width 0.2) (layer "B.Cu") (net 3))
 (segment (start 7.1 16.8) (end 6.7 16.4) (width 0.2) (layer "B.Cu") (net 3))
 (segment (start 9.2 20.8) (end 9.2 16.8) (width 0.2) (layer "B.Cu") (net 3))
 (segment (start 9 16.8) (end 7.1 16.8) (width 0.2) (layer "B.Cu") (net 3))
 (segment (start 5.6 19.2) (end 5.6 33.1) (width 0.2) (layer "F.Cu") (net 16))
 (segment (start 5.6 33.1) (end 1.7 37) (width 0.2) (layer "F.Cu") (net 16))
 (segment (start 4.8 18.4) (end 5.6 19.2) (width 0.2) (layer "F.Cu") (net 16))
 (segment (start 4.8 18.2) (end 4.8 18.4) (width 0.2) (layer "F.Cu") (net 16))
 (segment (start 19.1 5.3) (end 22.9 5.3) (width 0.2) (layer "F.Cu") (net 15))
 (segment (start 22.9 5.3) (end 34 16.4) (width 0.2) (layer "F.Cu") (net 15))
 (segment (start 18.8 9.5) (end 18.8 5.6) (width 0.2) (layer "F.Cu") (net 15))
 (segment (start 34.6 18.2) (end 35.6 18.2) (width 0.2) (layer "F.Cu") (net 15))
 (segment (start 35.6 18.2) (end 38.5 21.1) (width 0.2) (layer "F.Cu") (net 15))
 (segment (start 18.8 5.6) (end 19.1 5.3) (width 0.2) (layer "F.Cu") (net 15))
 (segment (start 38.5 21.1) (end 38.5 25) (width 0.2) (layer "F.Cu") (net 15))
 (segment (start 34 16.4) (end 34 17.6) (width 0.2) (layer "F.Cu") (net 15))
 (segment (start 34 17.6) (end 34.6 18.2) (width 0.2) (layer "F.Cu") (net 15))
 (segment (start 15.5 12.8) (end 18.8 9.5) (width 0.2) (layer "F.Cu") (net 15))
 (segment (start 35.8 29.6) (end 35.2 30.2) (width 0.2) (layer "F.Cu") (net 1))
 (segment (start 41.4 29.6) (end 35.8 29.6) (width 0.2) (layer "F.Cu") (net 1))
 (segment (start 35.2 30.2) (end 17.9 30.2) (width 0.2) (layer "F.Cu") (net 1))
 (segment (start 46 25) (end 41.4 29.6) (width 0.1998) (layer "F.Cu") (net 1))
 (segment (start 17.9 30.2) (end 15.1 33) (width 0.2) (layer "F.Cu") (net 1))
 (segment (start 45.1 29.1) (end 46 30) (width 0.2) (layer "F.Cu") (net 12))
 (segment (start 43.9 29.1) (end 45.1 29.1) (width 0.2) (layer "F.Cu") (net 12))
 (segment (start 40 33) (end 43.9 29.1) (width 0.2) (layer "F.Cu") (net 12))
 (segment (start 34.9 33) (end 40 33) (width 0.2) (layer "F.Cu") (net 12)))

